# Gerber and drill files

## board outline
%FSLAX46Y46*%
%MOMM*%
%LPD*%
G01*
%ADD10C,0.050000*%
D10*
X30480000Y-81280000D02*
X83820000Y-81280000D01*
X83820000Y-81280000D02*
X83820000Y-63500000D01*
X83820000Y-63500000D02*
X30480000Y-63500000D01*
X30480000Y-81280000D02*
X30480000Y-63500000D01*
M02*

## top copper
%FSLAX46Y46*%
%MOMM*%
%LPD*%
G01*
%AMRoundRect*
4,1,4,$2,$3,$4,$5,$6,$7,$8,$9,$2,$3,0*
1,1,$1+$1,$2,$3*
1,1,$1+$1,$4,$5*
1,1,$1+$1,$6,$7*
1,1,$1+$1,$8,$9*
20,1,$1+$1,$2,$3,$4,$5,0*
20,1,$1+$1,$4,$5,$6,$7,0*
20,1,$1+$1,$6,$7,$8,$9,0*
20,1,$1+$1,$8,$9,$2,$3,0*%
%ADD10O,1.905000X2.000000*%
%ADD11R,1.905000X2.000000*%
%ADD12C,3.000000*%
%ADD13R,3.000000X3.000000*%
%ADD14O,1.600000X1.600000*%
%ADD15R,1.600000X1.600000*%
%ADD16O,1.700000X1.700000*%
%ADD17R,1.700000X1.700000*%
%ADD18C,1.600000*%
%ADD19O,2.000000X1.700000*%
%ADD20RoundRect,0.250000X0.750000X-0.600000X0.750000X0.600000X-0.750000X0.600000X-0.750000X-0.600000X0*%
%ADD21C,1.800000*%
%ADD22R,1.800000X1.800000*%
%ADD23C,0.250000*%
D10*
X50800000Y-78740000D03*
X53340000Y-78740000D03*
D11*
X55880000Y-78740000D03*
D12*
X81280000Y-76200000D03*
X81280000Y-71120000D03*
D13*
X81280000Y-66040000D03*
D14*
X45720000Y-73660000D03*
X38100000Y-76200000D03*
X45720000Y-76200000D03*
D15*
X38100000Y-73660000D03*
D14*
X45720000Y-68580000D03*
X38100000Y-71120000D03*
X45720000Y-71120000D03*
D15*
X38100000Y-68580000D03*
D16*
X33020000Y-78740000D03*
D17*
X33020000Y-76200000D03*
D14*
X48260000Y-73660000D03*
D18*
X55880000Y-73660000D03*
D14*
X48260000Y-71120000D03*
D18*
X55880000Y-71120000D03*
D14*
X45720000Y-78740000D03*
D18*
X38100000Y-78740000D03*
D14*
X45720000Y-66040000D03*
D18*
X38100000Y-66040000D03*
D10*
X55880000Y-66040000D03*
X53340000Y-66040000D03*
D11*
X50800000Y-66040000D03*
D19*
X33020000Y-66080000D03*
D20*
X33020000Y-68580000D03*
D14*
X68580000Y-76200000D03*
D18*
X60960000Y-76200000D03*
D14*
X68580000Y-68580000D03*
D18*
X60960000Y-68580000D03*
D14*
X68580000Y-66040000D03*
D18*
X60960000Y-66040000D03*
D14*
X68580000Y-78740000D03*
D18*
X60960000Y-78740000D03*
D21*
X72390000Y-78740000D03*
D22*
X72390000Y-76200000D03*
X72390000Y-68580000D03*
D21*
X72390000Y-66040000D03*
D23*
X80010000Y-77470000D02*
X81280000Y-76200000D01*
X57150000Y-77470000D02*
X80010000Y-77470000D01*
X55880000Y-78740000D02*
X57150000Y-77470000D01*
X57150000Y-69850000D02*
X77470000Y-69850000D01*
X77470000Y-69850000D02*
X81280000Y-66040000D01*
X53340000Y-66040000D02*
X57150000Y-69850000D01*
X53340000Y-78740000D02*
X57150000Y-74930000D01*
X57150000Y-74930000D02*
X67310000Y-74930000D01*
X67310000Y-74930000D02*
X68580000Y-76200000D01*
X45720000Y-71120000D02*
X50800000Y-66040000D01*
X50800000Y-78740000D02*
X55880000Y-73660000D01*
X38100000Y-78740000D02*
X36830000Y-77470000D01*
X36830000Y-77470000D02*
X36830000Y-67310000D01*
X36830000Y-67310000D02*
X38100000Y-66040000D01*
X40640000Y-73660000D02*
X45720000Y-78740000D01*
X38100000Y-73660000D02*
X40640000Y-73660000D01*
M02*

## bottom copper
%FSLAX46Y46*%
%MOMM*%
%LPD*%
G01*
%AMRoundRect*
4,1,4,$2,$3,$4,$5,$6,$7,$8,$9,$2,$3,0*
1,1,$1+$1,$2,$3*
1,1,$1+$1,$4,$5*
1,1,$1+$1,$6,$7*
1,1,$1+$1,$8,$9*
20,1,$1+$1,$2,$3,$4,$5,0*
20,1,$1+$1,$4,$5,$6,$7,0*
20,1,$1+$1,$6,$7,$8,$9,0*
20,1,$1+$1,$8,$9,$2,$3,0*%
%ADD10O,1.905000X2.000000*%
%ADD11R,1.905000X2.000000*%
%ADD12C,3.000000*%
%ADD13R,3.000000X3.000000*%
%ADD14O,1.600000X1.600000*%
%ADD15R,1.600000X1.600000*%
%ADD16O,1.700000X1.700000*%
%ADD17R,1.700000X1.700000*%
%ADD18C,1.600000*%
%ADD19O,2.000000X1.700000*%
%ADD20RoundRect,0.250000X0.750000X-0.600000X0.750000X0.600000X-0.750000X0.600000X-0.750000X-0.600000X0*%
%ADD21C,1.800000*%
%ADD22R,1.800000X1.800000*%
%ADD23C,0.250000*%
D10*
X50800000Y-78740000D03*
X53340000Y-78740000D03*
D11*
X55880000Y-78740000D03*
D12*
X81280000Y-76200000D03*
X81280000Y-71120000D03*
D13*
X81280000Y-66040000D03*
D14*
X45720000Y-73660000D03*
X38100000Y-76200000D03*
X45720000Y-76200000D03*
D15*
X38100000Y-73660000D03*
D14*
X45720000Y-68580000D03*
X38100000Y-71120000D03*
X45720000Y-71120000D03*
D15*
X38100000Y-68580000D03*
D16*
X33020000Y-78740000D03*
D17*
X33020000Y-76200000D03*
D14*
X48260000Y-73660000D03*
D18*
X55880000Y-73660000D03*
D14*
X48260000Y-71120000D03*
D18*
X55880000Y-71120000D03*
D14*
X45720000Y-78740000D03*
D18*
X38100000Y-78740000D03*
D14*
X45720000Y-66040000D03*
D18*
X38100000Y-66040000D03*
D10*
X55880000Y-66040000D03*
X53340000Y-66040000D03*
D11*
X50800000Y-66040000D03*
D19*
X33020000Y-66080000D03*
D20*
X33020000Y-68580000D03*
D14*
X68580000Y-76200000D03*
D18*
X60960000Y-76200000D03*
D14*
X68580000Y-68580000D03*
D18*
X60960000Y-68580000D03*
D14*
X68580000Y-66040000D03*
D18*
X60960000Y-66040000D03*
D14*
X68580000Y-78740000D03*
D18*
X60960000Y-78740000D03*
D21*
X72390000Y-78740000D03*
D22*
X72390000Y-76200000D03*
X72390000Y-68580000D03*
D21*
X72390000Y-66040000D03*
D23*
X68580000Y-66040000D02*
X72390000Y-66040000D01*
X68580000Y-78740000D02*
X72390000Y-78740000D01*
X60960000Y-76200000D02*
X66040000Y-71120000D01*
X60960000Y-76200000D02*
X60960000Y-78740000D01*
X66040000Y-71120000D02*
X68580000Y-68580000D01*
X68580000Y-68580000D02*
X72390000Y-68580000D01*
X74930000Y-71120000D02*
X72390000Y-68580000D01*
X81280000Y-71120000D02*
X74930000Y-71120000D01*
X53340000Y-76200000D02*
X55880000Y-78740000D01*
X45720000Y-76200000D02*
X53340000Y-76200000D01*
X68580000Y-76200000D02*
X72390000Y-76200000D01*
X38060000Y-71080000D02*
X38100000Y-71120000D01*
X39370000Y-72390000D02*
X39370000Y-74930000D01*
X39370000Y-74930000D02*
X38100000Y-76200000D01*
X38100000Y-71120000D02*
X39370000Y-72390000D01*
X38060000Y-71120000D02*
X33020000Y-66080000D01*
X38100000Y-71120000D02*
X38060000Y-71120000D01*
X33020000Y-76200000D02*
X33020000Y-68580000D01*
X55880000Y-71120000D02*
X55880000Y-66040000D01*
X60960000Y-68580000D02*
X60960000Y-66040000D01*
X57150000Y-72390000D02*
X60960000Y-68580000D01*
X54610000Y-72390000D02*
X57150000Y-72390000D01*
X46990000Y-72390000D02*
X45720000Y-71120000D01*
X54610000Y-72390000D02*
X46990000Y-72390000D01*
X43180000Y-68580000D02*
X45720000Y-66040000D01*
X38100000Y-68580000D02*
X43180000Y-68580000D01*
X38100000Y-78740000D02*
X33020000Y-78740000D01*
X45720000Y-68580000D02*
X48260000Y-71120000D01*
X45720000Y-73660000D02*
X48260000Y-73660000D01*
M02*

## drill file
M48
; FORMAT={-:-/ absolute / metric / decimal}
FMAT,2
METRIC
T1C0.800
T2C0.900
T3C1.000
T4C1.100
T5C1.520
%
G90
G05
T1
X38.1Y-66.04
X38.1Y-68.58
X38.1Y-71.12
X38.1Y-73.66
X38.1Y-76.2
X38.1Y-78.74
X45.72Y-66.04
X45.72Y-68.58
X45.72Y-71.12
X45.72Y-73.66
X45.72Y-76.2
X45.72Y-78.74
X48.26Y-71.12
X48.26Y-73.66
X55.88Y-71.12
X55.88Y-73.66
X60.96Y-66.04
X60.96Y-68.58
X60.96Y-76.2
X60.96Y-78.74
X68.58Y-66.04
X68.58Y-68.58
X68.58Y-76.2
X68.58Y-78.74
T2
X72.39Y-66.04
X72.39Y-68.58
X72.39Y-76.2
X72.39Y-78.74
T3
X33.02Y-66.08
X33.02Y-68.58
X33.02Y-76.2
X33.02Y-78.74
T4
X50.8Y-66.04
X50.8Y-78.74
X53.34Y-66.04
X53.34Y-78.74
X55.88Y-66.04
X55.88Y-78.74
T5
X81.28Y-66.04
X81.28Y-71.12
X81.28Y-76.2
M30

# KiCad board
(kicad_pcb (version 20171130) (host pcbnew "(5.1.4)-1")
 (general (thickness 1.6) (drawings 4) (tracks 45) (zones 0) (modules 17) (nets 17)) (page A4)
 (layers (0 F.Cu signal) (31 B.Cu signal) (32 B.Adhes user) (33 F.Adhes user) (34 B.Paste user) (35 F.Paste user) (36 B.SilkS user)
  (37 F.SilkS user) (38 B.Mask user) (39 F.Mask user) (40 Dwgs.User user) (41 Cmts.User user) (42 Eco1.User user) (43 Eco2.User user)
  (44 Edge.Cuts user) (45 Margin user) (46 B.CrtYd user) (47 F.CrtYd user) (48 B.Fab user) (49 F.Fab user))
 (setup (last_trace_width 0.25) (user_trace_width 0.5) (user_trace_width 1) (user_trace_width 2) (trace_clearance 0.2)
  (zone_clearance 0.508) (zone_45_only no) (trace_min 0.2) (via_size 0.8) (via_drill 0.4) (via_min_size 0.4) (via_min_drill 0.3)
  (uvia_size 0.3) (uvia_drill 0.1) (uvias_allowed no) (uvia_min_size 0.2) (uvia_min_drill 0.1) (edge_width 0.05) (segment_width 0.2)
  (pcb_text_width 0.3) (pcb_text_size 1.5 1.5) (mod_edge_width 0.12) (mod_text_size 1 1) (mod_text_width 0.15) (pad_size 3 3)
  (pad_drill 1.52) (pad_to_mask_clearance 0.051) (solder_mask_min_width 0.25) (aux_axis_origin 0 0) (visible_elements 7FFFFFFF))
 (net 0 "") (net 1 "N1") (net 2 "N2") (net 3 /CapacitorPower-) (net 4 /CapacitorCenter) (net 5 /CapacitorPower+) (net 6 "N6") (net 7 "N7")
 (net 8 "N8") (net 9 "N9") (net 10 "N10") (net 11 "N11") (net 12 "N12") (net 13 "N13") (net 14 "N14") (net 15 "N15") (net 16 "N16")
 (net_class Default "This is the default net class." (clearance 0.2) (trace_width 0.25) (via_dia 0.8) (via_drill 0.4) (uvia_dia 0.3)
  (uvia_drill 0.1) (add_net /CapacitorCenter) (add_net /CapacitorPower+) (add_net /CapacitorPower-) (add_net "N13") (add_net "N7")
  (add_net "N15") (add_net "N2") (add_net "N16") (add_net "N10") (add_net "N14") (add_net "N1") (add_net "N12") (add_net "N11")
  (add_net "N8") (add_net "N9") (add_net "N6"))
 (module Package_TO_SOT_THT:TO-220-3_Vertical (layer F.Cu) (at 55.88 78.74 180)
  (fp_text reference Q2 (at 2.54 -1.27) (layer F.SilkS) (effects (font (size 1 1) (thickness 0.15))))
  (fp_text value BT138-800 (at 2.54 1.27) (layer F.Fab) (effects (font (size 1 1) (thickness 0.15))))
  (pad 3 thru_hole oval (at 5.08 0 180) (size 1.905 2) (drill 1.1) (layers *.Cu *.Mask) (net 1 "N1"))
  (pad 2 thru_hole oval (at 2.54 0 180) (size 1.905 2) (drill 1.1) (layers *.Cu *.Mask) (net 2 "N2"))
  (pad 1 thru_hole rect (at 0 0 180) (size 1.905 2) (drill 1.1) (layers *.Cu *.Mask) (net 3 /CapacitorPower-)))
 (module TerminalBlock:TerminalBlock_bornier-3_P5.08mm (layer F.Cu) (at 81.28 66.04 270)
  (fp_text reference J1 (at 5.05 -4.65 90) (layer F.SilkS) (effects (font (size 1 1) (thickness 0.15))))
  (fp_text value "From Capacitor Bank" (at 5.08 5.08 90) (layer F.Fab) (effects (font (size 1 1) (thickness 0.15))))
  (pad 3 thru_hole circle (at 10.16 0 270) (size 3 3) (drill 1.52) (layers *.Cu *.Mask) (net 3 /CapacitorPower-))
  (pad 2 thru_hole circle (at 5.08 0 270) (size 3 3) (drill 1.52) (layers *.Cu *.Mask) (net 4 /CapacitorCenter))
  (pad 1 thru_hole rect (at 0 0 270) (size 3 3) (drill 1.52) (layers *.Cu *.Mask) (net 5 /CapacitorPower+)))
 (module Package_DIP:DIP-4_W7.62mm (layer F.Cu) (at 38.1 73.66)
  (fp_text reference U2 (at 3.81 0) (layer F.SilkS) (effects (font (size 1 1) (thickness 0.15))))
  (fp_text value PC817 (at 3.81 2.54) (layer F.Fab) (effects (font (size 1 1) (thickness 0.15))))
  (pad 4 thru_hole oval (at 7.62 0) (size 1.6 1.6) (drill 0.8) (layers *.Cu *.Mask) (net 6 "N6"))
  (pad 2 thru_hole oval (at 0 2.54) (size 1.6 1.6) (drill 0.8) (layers *.Cu *.Mask) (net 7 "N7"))
  (pad 3 thru_hole oval (at 7.62 2.54) (size 1.6 1.6) (drill 0.8) (layers *.Cu *.Mask) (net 3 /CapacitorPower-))
  (pad 1 thru_hole rect (at 0 0) (size 1.6 1.6) (drill 0.8) (layers *.Cu *.Mask) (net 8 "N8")))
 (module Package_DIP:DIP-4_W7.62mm (layer F.Cu) (at 38.1 68.58)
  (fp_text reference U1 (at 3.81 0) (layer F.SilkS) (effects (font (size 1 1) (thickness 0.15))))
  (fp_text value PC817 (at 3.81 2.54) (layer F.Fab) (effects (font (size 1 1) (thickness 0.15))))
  (pad 4 thru_hole oval (at 7.62 0) (size 1.6 1.6) (drill 0.8) (layers *.Cu *.Mask) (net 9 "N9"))
  (pad 2 thru_hole oval (at 0 2.54) (size 1.6 1.6) (drill 0.8) (layers *.Cu *.Mask) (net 7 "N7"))
  (pad 3 thru_hole oval (at 7.62 2.54) (size 1.6 1.6) (drill 0.8) (layers *.Cu *.Mask) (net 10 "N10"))
  (pad 1 thru_hole rect (at 0 0) (size 1.6 1.6) (drill 0.8) (layers *.Cu *.Mask) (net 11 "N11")))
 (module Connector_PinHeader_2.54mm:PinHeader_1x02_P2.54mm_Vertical (layer F.Cu) (at 33.02 76.2)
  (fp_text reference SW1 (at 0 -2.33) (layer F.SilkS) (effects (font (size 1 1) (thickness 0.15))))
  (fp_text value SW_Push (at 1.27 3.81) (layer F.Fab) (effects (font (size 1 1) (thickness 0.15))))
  (pad 2 thru_hole oval (at 0 2.54) (size 1.7 1.7) (drill 1) (layers *.Cu *.Mask) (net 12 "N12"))
  (pad 1 thru_hole rect (at 0 0) (size 1.7 1.7) (drill 1) (layers *.Cu *.Mask) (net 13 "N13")))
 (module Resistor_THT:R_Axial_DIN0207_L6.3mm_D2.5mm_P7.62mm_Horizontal (layer F.Cu) (at 55.88 73.66 180)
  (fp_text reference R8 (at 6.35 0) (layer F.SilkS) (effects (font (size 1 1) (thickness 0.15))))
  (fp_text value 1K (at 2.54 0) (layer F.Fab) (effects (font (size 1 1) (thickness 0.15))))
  (pad 2 thru_hole oval (at 7.62 0 180) (size 1.6 1.6) (drill 0.8) (layers *.Cu *.Mask) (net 6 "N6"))
  (pad 1 thru_hole circle (at 0 0 180) (size 1.6 1.6) (drill 0.8) (layers *.Cu *.Mask) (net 1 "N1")))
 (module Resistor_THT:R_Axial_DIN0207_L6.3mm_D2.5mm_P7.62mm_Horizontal (layer F.Cu) (at 55.88 71.12 180)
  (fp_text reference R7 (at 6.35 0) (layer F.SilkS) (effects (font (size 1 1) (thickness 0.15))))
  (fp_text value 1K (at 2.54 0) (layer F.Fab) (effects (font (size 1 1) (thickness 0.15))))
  (pad 2 thru_hole oval (at 7.62 0 180) (size 1.6 1.6) (drill 0.8) (layers *.Cu *.Mask) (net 9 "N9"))
  (pad 1 thru_hole circle (at 0 0 180) (size 1.6 1.6) (drill 0.8) (layers *.Cu *.Mask) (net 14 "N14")))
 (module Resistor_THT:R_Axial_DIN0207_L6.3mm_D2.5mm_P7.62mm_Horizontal (layer F.Cu) (at 38.1 78.74)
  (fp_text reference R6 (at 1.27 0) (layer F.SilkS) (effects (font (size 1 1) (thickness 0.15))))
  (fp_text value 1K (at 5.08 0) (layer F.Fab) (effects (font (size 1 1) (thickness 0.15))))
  (pad 2 thru_hole oval (at 7.62 0) (size 1.6 1.6) (drill 0.8) (layers *.Cu *.Mask) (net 8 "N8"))
  (pad 1 thru_hole circle (at 0 0) (size 1.6 1.6) (drill 0.8) (layers *.Cu *.Mask) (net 12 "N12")))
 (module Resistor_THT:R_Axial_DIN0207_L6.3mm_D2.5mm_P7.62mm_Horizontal (layer F.Cu) (at 38.1 66.04)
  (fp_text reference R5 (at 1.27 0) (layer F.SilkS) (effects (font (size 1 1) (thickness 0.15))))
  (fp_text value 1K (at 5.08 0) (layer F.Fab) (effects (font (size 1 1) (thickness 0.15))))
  (pad 2 thru_hole oval (at 7.62 0) (size 1.6 1.6) (drill 0.8) (layers *.Cu *.Mask) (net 11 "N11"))
  (pad 1 thru_hole circle (at 0 0) (size 1.6 1.6) (drill 0.8) (layers *.Cu *.Mask) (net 12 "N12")))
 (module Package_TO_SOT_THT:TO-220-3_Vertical (layer F.Cu) (at 50.8 66.04)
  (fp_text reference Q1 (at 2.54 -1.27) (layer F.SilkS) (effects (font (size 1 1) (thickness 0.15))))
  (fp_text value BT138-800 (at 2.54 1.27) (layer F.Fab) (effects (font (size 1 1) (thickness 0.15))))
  (pad 3 thru_hole oval (at 5.08 0) (size 1.905 2) (drill 1.1) (layers *.Cu *.Mask) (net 14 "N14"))
  (pad 2 thru_hole oval (at 2.54 0) (size 1.905 2) (drill 1.1) (layers *.Cu *.Mask) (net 5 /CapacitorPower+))
  (pad 1 thru_hole rect (at 0 0) (size 1.905 2) (drill 1.1) (layers *.Cu *.Mask) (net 10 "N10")))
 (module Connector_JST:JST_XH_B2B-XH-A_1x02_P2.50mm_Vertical (layer F.Cu) (at 33.02 68.58 90)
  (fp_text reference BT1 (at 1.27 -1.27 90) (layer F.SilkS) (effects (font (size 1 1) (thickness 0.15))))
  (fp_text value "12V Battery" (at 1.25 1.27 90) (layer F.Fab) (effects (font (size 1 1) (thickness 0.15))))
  (pad 2 thru_hole oval (at 2.5 0 90) (size 1.7 2) (drill 1) (layers *.Cu *.Mask) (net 7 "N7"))
  (pad 1 thru_hole roundrect (at 0 0 90) (size 1.7 2) (drill 1) (layers *.Cu *.Mask) (roundrect_rratio 0.147059) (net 13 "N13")))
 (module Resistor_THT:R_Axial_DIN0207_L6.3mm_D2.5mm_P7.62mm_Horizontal (layer F.Cu) (at 60.96 76.2)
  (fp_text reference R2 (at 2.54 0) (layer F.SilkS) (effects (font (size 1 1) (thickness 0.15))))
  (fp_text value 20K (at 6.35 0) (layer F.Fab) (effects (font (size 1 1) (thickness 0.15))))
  (pad 2 thru_hole oval (at 7.62 0) (size 1.6 1.6) (drill 0.8) (layers *.Cu *.Mask) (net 2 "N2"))
  (pad 1 thru_hole circle (at 0 0) (size 1.6 1.6) (drill 0.8) (layers *.Cu *.Mask) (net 4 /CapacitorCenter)))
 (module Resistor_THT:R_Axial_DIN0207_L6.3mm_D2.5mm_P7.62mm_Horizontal (layer F.Cu) (at 60.96 68.58)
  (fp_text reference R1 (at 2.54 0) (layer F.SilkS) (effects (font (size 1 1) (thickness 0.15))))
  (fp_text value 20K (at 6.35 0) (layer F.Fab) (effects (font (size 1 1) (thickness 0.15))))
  (pad 2 thru_hole oval (at 7.62 0) (size 1.6 1.6) (drill 0.8) (layers *.Cu *.Mask) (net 4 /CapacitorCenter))
  (pad 1 thru_hole circle (at 0 0) (size 1.6 1.6) (drill 0.8) (layers *.Cu *.Mask) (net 10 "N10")))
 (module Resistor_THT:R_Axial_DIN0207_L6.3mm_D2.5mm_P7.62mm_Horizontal (layer F.Cu) (at 60.96 66.04)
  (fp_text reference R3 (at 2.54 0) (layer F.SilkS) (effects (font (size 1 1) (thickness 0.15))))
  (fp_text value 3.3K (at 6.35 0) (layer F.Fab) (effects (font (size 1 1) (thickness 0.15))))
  (pad 2 thru_hole oval (at 7.62 0) (size 1.6 1.6) (drill 0.8) (layers *.Cu *.Mask) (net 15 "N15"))
  (pad 1 thru_hole circle (at 0 0) (size 1.6 1.6) (drill 0.8) (layers *.Cu *.Mask) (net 10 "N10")))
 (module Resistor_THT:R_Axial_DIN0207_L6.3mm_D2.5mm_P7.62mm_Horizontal (layer F.Cu) (at 60.96 78.74)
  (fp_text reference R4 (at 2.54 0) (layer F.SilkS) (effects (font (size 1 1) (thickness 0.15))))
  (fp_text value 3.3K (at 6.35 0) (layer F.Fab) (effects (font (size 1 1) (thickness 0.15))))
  (pad 2 thru_hole oval (at 7.62 0) (size 1.6 1.6) (drill 0.8) (layers *.Cu *.Mask) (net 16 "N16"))
  (pad 1 thru_hole circle (at 0 0) (size 1.6 1.6) (drill 0.8) (layers *.Cu *.Mask) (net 4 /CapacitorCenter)))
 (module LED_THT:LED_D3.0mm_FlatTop (layer F.Cu) (at 72.39 76.2 270)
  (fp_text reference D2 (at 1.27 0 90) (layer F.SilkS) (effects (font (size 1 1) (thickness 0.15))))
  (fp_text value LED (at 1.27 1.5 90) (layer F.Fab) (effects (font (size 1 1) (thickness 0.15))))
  (pad 2 thru_hole circle (at 2.54 0 270) (size 1.8 1.8) (drill 0.9) (layers *.Cu *.Mask) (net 16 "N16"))
  (pad 1 thru_hole rect (at 0 0 270) (size 1.8 1.8) (drill 0.9) (layers *.Cu *.Mask) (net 2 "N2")))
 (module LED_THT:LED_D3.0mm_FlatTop (layer F.Cu) (at 72.39 68.58 90)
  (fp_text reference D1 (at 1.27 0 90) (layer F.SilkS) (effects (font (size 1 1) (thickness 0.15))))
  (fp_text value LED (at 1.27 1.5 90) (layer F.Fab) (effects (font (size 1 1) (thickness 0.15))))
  (pad 1 thru_hole rect (at 0 0 90) (size 1.8 1.8) (drill 0.9) (layers *.Cu *.Mask) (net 4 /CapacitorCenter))
  (pad 2 thru_hole circle (at 2.54 0 90) (size 1.8 1.8) (drill 0.9) (layers *.Cu *.Mask) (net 15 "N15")))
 (gr_line (start 30.48 81.28) (end 83.82 81.28) (layer Edge.Cuts) (width 0.05))
 (gr_line (start 83.82 81.28) (end 83.82 63.5) (layer Edge.Cuts) (width 0.05))
 (gr_line (start 83.82 63.5) (end 30.48 63.5) (layer Edge.Cuts) (width 0.05))
 (gr_line (start 30.48 81.28) (end 30.48 63.5) (layer Edge.Cuts) (width 0.05))
 (segment (start 68.58 66.04) (end 72.39 66.04) (width 0.25) (layer B.Cu) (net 15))
 (segment (start 68.58 78.74) (end 72.39 78.74) (width 0.25) (layer B.Cu) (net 16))
 (segment (start 60.96 76.2) (end 66.04 71.12) (width 0.25) (layer B.Cu) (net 4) (status 10))
 (segment (start 60.96 76.2) (end 60.96 78.74) (width 0.25) (layer B.Cu) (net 4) (status 30))
 (segment (start 66.04 71.12) (end 68.58 68.58) (width 0.25) (layer B.Cu) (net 4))
 (segment (start 68.58 68.58) (end 72.39 68.58) (width 0.25) (layer B.Cu) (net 4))
 (segment (start 74.93 71.12) (end 72.39 68.58) (width 0.25) (layer B.Cu) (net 4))
 (segment (start 81.28 71.12) (end 74.93 71.12) (width 0.25) (layer B.Cu) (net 4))
 (segment (start 53.34 76.2) (end 55.88 78.74) (width 0.25) (layer B.Cu) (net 3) (status 20))
 (segment (start 45.72 76.2) (end 53.34 76.2) (width 0.25) (layer B.Cu) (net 3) (status 10))
 (segment (start 80.01 77.47) (end 81.28 76.2) (width 0.25) (layer F.Cu) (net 3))
 (segment (start 57.15 77.47) (end 80.01 77.47) (width 0.25) (layer F.Cu) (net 3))
 (segment (start 55.88 78.74) (end 57.15 77.47) (width 0.25) (layer F.Cu) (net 3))
 (segment (start 57.15 69.85) (end 77.47 69.85) (width 0.25) (layer F.Cu) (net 5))
 (segment (start 77.47 69.85) (end 81.28 66.04) (width 0.25) (layer F.Cu) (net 5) (status 20))
 (segment (start 53.34 66.04) (end 57.15 69.85) (width 0.25) (layer F.Cu) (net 5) (status 10))
 (segment (start 68.58 76.2) (end 72.39 76.2) (width 0.25) (layer B.Cu) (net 2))
 (segment (start 53.34 78.74) (end 57.15 74.93) (width 0.25) (layer F.Cu) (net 2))
 (segment (start 57.15 74.93) (end 67.31 74.93) (width 0.25) (layer F.Cu) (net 2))
 (segment (start 67.31 74.93) (end 68.58 76.2) (width 0.25) (layer F.Cu) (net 2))
 (segment (start 38.06 71.08) (end 38.1 71.12) (width 0.25) (layer B.Cu) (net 7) (status 30))
 (segment (start 39.37 72.39) (end 39.37 74.93) (width 0.25) (layer B.Cu) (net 7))
 (segment (start 39.37 74.93) (end 38.1 76.2) (width 0.25) (layer B.Cu) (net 7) (status 20))
 (segment (start 38.1 71.12) (end 39.37 72.39) (width 0.25) (layer B.Cu) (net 7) (status 10))
 (segment (start 38.06 71.12) (end 33.02 66.08) (width 0.25) (layer B.Cu) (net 7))
 (segment (start 38.1 71.12) (end 38.06 71.12) (width 0.25) (layer B.Cu) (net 7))
 (segment (start 33.02 76.2) (end 33.02 68.58) (width 0.25) (layer B.Cu) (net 13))
 (segment (start 55.88 71.12) (end 55.88 66.04) (width 0.25) (layer B.Cu) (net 14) (status 30))
 (segment (start 45.72 71.12) (end 50.8 66.04) (width 0.25) (layer F.Cu) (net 10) (status 30))
 (segment (start 60.96 68.58) (end 60.96 66.04) (width 0.25) (layer B.Cu) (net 10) (status 30))
 (segment (start 57.15 72.39) (end 60.96 68.58) (width 0.25) (layer B.Cu) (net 10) (status 20))
 (segment (start 54.61 72.39) (end 57.15 72.39) (width 0.25) (layer B.Cu) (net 10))
 (segment (start 46.99 72.39) (end 45.72 71.12) (width 0.25) (layer B.Cu) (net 10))
 (segment (start 54.61 72.39) (end 46.99 72.39) (width 0.25) (layer B.Cu) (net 10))
 (segment (start 50.8 78.74) (end 55.88 73.66) (width 0.25) (layer F.Cu) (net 1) (status 30))
 (segment (start 43.18 68.58) (end 45.72 66.04) (width 0.25) (layer B.Cu) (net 11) (status 20))
 (segment (start 38.1 68.58) (end 43.18 68.58) (width 0.25) (layer B.Cu) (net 11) (status 10))
 (segment (start 38.1 78.74) (end 33.02 78.74) (width 0.25) (layer B.Cu) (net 12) (status 30))
 (segment (start 38.1 78.74) (end 36.83 77.47) (width 0.25) (layer F.Cu) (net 12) (status 10))
 (segment (start 36.83 77.47) (end 36.83 67.31) (width 0.25) (layer F.Cu) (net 12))
 (segment (start 36.83 67.31) (end 38.1 66.04) (width 0.25) (layer F.Cu) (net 12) (status 20))
 (segment (start 40.64 73.66) (end 45.72 78.74) (width 0.25) (layer F.Cu) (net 8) (status 20))
 (segment (start 38.1 73.66) (end 40.64 73.66) (width 0.25) (layer F.Cu) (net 8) (status 10))
 (segment (start 45.72 68.58) (end 48.26 71.12) (width 0.25) (layer B.Cu) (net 9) (status 30))
 (segment (start 45.72 73.66) (end 48.26 73.66) (width 0.25) (layer B.Cu) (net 6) (status 30)))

